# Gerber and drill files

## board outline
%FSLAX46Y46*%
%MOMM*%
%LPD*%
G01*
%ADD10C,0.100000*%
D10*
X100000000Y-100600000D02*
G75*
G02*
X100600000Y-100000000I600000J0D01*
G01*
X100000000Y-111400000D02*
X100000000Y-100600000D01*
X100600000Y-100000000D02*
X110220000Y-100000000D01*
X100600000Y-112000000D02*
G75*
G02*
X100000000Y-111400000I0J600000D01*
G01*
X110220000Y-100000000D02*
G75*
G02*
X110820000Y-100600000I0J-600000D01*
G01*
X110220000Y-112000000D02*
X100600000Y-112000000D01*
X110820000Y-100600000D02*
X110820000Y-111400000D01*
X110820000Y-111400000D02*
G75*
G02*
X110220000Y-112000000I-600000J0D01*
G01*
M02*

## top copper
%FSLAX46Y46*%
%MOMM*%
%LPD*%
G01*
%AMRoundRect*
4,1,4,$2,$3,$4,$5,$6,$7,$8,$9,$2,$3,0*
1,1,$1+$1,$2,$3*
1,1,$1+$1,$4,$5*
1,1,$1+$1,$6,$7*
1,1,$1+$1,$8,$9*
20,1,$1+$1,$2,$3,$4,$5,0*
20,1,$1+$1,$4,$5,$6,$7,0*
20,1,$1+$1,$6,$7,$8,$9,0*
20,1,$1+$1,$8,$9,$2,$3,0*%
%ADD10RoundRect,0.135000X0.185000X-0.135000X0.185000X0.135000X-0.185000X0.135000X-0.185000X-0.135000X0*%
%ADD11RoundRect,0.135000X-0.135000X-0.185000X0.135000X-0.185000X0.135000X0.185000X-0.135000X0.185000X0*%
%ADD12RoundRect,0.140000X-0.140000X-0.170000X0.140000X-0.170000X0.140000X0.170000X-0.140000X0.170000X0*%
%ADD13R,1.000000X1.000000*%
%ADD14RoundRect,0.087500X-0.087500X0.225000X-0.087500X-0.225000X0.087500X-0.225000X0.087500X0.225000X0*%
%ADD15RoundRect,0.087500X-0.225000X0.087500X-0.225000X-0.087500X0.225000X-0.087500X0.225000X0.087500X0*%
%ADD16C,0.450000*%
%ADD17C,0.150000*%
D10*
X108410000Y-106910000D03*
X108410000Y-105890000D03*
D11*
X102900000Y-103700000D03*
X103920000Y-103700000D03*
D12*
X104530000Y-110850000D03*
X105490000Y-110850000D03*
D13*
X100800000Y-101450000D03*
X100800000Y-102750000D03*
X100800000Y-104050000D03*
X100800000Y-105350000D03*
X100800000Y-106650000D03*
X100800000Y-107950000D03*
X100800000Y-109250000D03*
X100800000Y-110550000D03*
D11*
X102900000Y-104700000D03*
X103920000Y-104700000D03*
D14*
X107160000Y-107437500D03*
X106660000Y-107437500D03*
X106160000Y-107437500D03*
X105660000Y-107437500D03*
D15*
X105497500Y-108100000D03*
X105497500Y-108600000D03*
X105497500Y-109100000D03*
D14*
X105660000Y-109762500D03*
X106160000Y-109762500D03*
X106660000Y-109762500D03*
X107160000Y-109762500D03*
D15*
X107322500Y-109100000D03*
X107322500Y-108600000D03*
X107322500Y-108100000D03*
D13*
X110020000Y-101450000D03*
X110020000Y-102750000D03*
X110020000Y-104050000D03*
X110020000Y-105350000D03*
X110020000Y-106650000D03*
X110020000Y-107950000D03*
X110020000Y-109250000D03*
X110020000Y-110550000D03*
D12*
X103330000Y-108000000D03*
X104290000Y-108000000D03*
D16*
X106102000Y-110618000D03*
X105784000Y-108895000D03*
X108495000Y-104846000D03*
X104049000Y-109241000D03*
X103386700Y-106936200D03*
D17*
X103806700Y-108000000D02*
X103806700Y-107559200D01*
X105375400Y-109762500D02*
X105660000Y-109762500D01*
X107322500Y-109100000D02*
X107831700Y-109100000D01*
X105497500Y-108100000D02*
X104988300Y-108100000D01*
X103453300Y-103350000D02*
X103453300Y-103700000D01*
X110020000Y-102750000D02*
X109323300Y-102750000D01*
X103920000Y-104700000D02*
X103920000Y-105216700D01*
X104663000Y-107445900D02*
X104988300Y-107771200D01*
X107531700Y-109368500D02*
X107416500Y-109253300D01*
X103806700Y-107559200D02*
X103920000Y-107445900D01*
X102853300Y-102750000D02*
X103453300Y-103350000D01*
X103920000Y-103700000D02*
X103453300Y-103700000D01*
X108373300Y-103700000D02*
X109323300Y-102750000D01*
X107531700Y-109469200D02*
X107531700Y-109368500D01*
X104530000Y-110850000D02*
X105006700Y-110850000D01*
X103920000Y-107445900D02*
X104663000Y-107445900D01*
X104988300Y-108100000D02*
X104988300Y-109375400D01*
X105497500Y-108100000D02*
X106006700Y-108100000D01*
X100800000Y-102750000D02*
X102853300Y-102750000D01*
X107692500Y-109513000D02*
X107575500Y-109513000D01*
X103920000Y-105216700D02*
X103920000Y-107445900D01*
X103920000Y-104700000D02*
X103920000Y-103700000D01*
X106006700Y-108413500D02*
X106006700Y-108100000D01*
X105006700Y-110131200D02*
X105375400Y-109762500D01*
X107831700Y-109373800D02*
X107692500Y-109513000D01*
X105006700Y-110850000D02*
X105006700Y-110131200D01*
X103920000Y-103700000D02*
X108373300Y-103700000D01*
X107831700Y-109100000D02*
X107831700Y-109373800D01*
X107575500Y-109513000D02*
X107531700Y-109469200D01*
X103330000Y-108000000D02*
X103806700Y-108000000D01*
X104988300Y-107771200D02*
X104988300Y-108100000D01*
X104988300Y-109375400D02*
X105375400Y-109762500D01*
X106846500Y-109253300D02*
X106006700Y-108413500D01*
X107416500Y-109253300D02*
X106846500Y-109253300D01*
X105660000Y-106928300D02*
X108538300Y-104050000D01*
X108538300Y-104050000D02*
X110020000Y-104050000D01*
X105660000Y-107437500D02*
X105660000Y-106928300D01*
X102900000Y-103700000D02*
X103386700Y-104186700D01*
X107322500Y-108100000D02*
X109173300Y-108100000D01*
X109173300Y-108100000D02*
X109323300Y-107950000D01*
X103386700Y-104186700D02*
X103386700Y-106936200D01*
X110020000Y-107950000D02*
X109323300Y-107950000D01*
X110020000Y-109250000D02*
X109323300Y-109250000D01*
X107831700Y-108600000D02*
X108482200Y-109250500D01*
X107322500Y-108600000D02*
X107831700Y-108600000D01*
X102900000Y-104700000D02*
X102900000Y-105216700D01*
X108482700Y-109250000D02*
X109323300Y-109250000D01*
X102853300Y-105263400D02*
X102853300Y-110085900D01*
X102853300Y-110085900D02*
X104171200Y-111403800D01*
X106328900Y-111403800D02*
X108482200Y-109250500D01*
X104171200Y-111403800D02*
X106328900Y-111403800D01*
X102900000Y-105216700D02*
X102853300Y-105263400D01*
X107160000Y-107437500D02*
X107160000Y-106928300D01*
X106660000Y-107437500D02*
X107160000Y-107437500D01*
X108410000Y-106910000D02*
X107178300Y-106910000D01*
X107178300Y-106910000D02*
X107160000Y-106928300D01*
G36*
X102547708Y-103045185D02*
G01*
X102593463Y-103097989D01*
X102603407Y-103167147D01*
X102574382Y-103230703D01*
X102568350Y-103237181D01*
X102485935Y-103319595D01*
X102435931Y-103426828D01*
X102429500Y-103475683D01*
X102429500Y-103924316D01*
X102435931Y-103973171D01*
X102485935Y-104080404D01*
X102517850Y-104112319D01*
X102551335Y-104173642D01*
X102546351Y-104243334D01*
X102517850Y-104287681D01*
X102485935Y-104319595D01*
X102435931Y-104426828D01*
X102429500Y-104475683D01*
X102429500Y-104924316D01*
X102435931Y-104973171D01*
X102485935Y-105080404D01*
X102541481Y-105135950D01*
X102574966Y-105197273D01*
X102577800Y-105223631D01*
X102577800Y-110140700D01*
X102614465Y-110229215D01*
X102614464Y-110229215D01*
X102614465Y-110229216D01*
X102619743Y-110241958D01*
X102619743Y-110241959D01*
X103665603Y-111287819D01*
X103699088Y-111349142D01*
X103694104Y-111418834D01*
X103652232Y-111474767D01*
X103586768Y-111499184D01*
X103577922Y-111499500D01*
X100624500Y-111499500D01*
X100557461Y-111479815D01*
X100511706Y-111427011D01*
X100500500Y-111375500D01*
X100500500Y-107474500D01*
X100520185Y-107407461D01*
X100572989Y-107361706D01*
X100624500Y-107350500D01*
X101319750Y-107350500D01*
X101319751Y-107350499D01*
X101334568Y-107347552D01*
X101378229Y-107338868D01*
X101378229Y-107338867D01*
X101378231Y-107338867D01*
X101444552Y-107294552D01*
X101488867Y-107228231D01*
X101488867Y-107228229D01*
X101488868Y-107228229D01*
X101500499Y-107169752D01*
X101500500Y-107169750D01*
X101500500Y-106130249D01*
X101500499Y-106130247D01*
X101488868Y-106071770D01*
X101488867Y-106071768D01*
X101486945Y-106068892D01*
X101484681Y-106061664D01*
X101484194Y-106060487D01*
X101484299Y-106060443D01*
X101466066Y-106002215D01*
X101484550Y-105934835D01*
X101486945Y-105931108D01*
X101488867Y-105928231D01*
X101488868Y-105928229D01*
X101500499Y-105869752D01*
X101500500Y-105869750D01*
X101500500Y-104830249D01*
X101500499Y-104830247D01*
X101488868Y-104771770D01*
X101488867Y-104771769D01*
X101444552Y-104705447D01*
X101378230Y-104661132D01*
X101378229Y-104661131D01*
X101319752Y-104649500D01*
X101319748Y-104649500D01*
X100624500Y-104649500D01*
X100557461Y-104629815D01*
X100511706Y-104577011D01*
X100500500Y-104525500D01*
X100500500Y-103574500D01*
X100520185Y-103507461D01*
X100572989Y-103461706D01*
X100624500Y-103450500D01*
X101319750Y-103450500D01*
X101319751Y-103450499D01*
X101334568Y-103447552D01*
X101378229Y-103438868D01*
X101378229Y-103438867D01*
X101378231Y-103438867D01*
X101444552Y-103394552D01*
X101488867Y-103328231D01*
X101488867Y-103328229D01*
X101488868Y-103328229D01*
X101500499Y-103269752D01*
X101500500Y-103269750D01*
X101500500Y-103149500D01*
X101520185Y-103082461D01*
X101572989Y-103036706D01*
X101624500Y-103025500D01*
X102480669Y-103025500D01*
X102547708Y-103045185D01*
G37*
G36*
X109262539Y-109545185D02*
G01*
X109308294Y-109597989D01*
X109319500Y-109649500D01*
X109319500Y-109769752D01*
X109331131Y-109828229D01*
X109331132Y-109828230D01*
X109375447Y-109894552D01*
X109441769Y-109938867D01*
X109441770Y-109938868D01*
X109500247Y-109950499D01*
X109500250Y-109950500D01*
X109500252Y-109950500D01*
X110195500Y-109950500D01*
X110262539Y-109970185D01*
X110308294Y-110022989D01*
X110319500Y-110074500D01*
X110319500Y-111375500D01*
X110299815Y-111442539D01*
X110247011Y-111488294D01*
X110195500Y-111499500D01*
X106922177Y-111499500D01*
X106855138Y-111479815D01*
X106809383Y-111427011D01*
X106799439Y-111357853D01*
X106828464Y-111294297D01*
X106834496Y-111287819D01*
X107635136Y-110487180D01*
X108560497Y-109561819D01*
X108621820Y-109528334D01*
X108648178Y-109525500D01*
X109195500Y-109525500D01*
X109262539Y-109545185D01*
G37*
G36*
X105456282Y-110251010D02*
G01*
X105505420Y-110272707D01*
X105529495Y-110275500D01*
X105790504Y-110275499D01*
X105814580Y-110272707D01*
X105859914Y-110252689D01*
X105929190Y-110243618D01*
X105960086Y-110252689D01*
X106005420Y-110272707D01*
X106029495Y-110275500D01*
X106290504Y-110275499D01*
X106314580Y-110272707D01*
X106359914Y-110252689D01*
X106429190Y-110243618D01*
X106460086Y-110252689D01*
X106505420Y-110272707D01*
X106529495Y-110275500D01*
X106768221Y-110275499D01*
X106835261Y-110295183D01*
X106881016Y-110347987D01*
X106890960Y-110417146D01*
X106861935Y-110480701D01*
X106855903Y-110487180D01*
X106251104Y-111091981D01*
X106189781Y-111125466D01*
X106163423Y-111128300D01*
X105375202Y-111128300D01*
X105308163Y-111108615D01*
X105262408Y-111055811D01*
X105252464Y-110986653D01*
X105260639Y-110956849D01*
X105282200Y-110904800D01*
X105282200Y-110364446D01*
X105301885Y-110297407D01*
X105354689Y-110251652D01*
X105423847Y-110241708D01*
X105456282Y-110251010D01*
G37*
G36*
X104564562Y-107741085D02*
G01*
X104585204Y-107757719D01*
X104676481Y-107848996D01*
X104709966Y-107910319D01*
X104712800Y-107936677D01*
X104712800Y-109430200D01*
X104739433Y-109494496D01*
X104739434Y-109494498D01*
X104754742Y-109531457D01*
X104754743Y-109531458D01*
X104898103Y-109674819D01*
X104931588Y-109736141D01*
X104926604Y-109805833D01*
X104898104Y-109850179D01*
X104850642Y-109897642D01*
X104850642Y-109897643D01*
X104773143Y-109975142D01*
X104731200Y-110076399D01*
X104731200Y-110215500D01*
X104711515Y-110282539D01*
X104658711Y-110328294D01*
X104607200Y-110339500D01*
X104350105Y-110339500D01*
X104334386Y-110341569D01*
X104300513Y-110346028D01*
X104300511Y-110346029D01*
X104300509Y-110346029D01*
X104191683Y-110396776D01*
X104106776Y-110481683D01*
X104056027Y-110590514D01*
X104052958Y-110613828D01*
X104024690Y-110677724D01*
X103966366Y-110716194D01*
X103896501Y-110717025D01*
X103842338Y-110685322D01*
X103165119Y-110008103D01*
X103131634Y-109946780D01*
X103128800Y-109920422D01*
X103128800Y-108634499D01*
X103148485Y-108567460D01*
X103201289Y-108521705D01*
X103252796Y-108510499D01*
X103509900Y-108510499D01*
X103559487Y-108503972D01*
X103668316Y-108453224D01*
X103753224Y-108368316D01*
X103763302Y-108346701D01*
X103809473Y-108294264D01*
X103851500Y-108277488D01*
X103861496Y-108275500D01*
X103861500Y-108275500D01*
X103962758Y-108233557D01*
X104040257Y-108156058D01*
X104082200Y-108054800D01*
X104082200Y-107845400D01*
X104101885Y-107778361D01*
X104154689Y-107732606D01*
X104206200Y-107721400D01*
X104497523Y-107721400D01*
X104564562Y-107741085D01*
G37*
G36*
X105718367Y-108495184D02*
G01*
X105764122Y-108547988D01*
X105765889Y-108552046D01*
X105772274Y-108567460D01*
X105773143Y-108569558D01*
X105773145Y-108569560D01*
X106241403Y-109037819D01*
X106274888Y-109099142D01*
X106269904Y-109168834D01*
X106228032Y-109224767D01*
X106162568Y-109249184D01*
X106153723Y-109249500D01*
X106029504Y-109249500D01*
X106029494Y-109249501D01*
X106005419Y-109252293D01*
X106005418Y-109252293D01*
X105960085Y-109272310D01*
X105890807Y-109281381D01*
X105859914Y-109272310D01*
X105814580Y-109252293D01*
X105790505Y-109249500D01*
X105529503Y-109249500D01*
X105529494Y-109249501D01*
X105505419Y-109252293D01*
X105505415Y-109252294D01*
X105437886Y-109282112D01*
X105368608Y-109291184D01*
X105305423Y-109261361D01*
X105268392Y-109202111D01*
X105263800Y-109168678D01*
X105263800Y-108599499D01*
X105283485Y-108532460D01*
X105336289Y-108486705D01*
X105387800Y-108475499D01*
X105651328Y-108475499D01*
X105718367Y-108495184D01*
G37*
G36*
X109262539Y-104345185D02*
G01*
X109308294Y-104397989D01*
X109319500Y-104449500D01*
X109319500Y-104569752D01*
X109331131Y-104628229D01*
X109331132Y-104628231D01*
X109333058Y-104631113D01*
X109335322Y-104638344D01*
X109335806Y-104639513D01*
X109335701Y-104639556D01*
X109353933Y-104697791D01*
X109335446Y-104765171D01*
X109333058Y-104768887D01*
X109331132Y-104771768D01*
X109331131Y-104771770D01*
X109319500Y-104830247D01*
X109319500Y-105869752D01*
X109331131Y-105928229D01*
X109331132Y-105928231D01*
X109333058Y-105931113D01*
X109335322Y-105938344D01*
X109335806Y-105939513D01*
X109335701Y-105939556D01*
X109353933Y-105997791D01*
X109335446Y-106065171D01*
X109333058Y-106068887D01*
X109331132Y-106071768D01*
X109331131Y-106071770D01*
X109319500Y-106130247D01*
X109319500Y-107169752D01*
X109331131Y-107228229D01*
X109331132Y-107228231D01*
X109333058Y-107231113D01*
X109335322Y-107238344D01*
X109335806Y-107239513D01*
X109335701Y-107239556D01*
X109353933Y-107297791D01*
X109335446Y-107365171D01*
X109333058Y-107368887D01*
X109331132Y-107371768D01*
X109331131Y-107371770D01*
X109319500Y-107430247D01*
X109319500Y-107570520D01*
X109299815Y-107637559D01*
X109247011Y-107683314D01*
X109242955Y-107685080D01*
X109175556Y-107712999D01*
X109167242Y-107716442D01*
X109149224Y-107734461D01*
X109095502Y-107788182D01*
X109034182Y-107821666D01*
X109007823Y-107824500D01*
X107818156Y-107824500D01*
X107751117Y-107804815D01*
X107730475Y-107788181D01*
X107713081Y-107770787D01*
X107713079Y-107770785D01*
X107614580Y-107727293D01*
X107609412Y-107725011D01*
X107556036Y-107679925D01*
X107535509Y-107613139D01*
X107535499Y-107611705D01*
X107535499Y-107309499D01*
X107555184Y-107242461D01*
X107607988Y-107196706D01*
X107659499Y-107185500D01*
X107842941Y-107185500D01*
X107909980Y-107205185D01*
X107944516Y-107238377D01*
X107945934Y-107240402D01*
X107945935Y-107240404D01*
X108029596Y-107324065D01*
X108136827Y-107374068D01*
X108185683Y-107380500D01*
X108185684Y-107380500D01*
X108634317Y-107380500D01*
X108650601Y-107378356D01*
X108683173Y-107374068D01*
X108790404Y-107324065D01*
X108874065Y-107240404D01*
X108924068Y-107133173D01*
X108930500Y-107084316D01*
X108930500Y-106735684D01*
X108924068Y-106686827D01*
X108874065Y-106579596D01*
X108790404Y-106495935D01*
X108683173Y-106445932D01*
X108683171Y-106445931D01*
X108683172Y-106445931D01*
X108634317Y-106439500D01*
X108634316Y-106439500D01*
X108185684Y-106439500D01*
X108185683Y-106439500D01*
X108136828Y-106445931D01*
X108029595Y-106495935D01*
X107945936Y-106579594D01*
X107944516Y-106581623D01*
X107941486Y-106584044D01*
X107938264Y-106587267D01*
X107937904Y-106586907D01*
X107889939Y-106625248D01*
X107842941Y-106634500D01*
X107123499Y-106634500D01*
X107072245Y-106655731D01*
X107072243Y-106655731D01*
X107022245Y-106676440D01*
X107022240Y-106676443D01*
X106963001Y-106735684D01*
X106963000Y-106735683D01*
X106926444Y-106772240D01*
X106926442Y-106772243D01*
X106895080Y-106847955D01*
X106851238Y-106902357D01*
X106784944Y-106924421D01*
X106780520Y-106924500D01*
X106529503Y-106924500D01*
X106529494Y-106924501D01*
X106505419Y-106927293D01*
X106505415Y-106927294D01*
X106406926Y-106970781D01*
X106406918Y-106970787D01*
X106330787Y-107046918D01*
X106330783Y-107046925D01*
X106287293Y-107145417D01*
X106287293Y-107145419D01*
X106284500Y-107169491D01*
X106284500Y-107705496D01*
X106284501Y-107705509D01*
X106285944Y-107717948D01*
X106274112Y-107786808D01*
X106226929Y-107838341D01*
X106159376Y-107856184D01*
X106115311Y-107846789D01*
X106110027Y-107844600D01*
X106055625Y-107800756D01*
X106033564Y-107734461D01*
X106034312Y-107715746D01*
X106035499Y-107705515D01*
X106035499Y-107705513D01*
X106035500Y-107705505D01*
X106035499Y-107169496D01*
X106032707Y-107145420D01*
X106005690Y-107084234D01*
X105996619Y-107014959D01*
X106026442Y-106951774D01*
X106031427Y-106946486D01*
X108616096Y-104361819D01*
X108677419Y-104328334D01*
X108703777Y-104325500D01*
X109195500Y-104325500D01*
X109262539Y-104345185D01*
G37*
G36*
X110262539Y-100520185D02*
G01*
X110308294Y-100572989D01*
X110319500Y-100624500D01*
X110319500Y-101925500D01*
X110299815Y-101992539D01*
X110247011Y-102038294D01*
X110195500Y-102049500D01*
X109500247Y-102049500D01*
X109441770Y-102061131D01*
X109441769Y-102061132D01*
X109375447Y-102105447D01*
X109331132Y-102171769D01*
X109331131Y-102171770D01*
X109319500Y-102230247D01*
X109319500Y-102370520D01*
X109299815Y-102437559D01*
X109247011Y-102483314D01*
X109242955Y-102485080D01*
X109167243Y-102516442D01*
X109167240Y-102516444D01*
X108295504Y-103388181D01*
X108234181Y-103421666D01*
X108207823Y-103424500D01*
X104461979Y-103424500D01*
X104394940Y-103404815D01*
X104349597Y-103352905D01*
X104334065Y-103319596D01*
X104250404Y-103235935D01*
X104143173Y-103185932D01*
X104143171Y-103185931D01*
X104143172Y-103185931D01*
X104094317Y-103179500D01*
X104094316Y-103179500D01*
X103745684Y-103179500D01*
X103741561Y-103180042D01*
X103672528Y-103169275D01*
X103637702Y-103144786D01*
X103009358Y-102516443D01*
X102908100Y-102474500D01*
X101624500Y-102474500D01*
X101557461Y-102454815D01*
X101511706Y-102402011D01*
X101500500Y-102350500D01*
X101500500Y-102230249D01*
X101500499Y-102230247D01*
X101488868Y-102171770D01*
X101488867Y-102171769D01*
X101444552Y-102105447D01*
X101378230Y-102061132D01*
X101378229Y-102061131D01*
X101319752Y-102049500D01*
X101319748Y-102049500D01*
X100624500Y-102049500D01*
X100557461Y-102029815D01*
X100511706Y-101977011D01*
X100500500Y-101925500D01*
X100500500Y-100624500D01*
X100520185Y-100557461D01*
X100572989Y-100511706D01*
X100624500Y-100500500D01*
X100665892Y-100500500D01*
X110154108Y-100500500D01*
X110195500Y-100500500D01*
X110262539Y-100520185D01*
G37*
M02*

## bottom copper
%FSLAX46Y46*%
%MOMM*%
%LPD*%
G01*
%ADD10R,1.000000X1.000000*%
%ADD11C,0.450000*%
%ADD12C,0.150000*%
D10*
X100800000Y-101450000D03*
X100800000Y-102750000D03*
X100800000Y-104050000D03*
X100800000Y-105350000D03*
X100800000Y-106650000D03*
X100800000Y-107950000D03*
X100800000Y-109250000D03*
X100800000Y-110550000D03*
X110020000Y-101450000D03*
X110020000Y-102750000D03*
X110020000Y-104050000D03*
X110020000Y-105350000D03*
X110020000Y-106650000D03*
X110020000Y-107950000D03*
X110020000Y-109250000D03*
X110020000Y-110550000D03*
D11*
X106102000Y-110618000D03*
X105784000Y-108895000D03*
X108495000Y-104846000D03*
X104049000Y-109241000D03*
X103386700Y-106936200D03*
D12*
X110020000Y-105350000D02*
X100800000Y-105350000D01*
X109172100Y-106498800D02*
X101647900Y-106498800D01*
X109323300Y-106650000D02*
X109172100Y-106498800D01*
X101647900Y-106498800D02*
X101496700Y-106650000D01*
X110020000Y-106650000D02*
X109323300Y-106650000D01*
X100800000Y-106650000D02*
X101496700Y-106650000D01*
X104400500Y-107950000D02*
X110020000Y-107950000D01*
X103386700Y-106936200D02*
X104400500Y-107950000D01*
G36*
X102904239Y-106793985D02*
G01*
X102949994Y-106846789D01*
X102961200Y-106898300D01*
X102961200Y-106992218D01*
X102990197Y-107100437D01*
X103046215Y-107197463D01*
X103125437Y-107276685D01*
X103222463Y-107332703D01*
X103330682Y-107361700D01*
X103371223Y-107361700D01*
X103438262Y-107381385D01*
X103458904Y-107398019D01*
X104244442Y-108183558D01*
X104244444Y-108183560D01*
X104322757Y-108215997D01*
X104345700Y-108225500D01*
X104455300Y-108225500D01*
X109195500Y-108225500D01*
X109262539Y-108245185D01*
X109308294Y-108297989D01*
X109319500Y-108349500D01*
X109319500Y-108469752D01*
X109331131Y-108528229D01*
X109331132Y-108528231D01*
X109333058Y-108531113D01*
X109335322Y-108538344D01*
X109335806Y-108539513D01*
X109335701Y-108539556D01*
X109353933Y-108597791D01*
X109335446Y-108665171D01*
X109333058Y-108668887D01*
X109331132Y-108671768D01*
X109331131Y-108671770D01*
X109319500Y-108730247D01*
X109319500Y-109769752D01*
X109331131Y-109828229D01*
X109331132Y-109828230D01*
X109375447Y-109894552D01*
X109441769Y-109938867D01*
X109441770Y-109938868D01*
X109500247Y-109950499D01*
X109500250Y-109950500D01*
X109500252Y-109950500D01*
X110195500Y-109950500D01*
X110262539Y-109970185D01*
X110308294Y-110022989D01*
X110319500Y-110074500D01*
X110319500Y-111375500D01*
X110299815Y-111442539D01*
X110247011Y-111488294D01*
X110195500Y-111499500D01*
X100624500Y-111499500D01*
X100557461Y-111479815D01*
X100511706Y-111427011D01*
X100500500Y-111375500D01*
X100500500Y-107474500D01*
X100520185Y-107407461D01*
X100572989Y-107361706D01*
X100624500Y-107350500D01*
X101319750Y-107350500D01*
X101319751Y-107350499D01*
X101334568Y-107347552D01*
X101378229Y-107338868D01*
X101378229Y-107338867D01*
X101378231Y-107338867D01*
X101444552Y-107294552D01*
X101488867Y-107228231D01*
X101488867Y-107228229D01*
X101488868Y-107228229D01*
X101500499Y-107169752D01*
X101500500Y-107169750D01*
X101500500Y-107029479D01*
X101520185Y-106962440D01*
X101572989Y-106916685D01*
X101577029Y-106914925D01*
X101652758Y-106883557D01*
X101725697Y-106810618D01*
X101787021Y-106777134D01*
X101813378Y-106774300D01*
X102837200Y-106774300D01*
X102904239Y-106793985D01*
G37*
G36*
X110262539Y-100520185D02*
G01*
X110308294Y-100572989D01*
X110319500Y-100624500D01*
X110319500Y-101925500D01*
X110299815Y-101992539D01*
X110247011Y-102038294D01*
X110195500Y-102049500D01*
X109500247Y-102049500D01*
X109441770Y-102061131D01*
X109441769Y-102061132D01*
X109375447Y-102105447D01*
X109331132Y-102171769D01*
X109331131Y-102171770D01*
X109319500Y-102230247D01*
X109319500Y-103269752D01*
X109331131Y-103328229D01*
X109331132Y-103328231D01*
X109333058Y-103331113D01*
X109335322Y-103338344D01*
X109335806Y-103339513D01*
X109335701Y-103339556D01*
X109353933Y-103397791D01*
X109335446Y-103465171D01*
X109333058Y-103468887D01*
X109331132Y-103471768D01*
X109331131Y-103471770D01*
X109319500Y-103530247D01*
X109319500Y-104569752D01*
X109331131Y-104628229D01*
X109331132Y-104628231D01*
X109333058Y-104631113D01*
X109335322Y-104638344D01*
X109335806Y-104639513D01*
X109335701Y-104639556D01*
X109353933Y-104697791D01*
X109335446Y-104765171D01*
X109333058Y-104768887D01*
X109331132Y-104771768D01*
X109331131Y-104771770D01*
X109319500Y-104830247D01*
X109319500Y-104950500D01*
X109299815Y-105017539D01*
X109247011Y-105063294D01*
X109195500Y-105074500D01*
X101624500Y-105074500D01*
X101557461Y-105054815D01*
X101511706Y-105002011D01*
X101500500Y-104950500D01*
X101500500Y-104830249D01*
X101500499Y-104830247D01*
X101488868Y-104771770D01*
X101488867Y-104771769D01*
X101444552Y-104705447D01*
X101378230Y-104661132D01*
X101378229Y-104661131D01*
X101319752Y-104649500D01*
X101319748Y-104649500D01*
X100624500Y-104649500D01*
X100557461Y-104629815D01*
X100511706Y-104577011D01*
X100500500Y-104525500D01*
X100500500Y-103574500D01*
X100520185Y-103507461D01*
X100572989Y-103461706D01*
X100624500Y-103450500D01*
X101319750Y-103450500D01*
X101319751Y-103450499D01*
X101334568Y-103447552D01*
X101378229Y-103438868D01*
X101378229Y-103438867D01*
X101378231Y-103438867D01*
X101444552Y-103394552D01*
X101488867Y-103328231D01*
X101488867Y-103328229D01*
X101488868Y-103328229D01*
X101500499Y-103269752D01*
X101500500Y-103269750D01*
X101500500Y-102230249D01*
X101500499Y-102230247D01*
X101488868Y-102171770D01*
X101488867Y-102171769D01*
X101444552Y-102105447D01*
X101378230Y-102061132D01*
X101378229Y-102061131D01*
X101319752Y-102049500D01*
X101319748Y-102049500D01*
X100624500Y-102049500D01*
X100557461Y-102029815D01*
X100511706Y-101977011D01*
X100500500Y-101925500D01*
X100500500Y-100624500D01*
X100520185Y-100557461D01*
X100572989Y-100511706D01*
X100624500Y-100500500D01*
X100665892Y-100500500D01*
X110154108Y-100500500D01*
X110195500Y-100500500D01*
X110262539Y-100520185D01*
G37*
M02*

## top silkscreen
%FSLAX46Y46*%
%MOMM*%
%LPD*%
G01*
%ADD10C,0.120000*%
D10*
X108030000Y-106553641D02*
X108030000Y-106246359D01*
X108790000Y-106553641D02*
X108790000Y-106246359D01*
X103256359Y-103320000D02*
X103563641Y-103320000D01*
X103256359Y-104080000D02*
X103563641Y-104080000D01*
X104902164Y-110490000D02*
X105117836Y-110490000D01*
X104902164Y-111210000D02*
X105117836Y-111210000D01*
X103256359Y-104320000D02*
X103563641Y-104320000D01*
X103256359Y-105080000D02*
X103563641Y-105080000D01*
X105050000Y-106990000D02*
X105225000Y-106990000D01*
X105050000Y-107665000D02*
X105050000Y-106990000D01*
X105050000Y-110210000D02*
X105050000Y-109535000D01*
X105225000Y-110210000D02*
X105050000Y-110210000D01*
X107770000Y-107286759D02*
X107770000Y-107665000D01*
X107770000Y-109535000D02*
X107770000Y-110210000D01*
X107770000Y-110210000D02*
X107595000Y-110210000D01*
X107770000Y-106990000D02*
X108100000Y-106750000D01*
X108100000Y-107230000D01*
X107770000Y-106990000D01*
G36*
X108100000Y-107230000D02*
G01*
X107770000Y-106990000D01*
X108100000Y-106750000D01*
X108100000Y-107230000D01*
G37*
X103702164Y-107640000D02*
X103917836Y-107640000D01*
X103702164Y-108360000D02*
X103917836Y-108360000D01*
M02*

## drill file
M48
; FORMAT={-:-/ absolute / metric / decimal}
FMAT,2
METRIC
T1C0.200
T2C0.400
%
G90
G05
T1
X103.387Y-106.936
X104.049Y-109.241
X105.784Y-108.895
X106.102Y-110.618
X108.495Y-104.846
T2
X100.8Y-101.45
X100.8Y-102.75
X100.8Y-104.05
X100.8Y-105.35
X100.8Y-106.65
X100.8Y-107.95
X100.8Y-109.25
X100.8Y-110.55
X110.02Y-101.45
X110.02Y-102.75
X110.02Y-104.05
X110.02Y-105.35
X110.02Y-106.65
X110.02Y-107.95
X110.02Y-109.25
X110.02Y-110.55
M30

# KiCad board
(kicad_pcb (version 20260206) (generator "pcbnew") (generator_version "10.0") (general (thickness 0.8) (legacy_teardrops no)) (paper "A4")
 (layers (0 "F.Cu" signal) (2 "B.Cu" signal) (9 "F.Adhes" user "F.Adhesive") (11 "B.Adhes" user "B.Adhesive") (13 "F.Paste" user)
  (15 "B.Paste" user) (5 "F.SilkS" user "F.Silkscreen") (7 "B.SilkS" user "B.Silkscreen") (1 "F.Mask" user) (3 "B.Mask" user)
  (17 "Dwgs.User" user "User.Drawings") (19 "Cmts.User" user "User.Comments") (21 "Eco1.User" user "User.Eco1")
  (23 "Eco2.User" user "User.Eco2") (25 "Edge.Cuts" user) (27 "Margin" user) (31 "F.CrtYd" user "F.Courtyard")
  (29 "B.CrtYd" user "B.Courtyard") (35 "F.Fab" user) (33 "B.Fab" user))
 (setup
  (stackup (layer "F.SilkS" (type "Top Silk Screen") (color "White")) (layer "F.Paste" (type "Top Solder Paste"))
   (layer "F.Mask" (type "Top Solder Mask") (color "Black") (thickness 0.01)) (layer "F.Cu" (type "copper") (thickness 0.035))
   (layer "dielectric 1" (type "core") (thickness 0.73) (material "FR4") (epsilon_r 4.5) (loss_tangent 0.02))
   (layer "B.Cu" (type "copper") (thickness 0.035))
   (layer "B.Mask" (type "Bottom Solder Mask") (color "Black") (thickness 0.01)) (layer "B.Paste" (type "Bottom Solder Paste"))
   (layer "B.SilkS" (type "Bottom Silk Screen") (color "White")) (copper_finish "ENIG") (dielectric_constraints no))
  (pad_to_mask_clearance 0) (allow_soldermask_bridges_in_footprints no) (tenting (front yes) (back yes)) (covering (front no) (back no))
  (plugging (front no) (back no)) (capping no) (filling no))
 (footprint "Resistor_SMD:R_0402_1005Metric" (layer "F.Cu") (at 108.41 106.4 90)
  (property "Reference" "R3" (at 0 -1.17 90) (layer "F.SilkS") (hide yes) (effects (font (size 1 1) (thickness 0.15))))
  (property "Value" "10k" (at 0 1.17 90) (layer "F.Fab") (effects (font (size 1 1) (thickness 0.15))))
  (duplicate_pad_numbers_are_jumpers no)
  (fp_line (start -0.153641 -0.38) (end 0.153641 -0.38) (stroke (width 0.12) (type solid)) (layer "F.SilkS"))
  (fp_line (start -0.153641 0.38) (end 0.153641 0.38) (stroke (width 0.12) (type solid)) (layer "F.SilkS"))
  (pad "1" smd roundrect (at -0.51 0 90) (size 0.54 0.64) (layers "F.Cu" "F.Mask" "F.Paste") (roundrect_rratio 0.25) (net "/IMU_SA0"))
  (pad "2" smd roundrect (at 0.51 0 90) (size 0.54 0.64) (layers "F.Cu" "F.Mask" "F.Paste") (roundrect_rratio 0.25) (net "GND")))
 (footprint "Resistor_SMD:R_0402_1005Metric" (layer "F.Cu") (at 103.41 103.7)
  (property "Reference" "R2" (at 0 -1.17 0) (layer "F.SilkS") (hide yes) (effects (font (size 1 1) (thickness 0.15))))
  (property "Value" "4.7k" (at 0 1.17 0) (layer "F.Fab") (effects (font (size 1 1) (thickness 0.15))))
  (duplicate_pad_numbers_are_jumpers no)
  (fp_line (start -0.153641 -0.38) (end 0.153641 -0.38) (stroke (width 0.12) (type solid)) (layer "F.SilkS"))
  (fp_line (start -0.153641 0.38) (end 0.153641 0.38) (stroke (width 0.12) (type solid)) (layer "F.SilkS"))
  (pad "1" smd roundrect (at -0.51 0) (size 0.54 0.64) (layers "F.Cu" "F.Mask" "F.Paste") (roundrect_rratio 0.25) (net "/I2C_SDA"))
  (pad "2" smd roundrect (at 0.51 0) (size 0.54 0.64) (layers "F.Cu" "F.Mask" "F.Paste") (roundrect_rratio 0.25) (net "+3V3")))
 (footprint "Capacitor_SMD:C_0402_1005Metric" (layer "F.Cu") (at 105.01 110.85)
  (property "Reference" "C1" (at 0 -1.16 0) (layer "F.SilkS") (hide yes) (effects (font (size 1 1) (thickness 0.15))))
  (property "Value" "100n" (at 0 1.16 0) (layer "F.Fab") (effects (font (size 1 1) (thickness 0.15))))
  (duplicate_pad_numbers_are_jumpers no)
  (fp_line (start -0.107836 -0.36) (end 0.107836 -0.36) (stroke (width 0.12) (type solid)) (layer "F.SilkS"))
  (fp_line (start -0.107836 0.36) (end 0.107836 0.36) (stroke (width 0.12) (type solid)) (layer "F.SilkS"))
  (pad "1" smd roundrect (at -0.48 0) (size 0.56 0.62) (layers "F.Cu" "F.Mask" "F.Paste") (roundrect_rratio 0.25) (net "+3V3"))
  (pad "2" smd roundrect (at 0.48 0) (size 0.56 0.62) (layers "F.Cu" "F.Mask" "F.Paste") (roundrect_rratio 0.25) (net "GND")))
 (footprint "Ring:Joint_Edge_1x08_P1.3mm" (layer "F.Cu") (at 100.8 106)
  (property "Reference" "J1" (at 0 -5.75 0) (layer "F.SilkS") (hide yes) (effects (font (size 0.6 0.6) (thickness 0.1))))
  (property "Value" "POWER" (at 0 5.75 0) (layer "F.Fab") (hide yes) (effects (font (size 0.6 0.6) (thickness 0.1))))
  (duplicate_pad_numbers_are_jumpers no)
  (pad "1" thru_hole rect (at 0 -4.55) (size 1 1) (drill 0.4) (layers "*.Cu" "*.Mask") (remove_unused_layers no) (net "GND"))
  (pad "2" thru_hole rect (at 0 -3.25) (size 1 1) (drill 0.4) (layers "*.Cu" "*.Mask") (remove_unused_layers no) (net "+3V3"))
  (pad "3" thru_hole rect (at 0 -1.95) (size 1 1) (drill 0.4) (layers "*.Cu" "*.Mask") (remove_unused_layers no) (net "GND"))
  (pad "4" thru_hole rect (at 0 -0.65) (size 1 1) (drill 0.4) (layers "*.Cu" "*.Mask") (remove_unused_layers no) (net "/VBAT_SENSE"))
  (pad "5" thru_hole rect (at 0 0.65) (size 1 1) (drill 0.4) (layers "*.Cu" "*.Mask") (remove_unused_layers no) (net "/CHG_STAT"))
  (pad "6" thru_hole rect (at 0 1.95) (size 1 1) (drill 0.4) (layers "*.Cu" "*.Mask") (remove_unused_layers no) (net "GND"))
  (pad "7" thru_hole rect (at 0 3.25) (size 1 1) (drill 0.4) (layers "*.Cu" "*.Mask") (remove_unused_layers no) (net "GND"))
  (pad "8" thru_hole rect (at 0 4.55) (size 1 1) (drill 0.4) (layers "*.Cu" "*.Mask") (remove_unused_layers no) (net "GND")))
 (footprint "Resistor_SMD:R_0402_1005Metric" (layer "F.Cu") (at 103.41 104.7)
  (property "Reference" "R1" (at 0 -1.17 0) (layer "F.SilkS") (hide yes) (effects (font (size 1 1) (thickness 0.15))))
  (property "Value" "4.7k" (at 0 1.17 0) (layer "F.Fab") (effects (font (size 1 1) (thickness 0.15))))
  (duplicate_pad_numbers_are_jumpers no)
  (fp_line (start -0.153641 -0.38) (end 0.153641 -0.38) (stroke (width 0.12) (type solid)) (layer "F.SilkS"))
  (fp_line (start -0.153641 0.38) (end 0.153641 0.38) (stroke (width 0.12) (type solid)) (layer "F.SilkS"))
  (pad "1" smd roundrect (at -0.51 0) (size 0.54 0.64) (layers "F.Cu" "F.Mask" "F.Paste") (roundrect_rratio 0.25) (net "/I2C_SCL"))
  (pad "2" smd roundrect (at 0.51 0) (size 0.54 0.64) (layers "F.Cu" "F.Mask" "F.Paste") (roundrect_rratio 0.25) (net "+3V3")))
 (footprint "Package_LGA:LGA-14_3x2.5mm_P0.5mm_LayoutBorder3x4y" (layer "F.Cu") (at 106.41 108.6 -90)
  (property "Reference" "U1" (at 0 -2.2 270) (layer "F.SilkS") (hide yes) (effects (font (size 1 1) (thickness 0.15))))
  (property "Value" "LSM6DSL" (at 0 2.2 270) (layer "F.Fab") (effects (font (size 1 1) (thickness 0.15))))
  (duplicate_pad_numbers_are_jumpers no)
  (fp_line (start -1.61 1.36) (end -1.61 1.185) (stroke (width 0.12) (type solid)) (layer "F.SilkS"))
  (fp_line (start -0.935 1.36) (end -1.61 1.36) (stroke (width 0.12) (type solid)) (layer "F.SilkS"))
  (fp_line (start 1.61 1.36) (end 0.935 1.36) (stroke (width 0.12) (type solid)) (layer "F.SilkS"))
  (fp_line (start 1.61 1.185) (end 1.61 1.36) (stroke (width 0.12) (type solid)) (layer "F.SilkS"))
  (fp_line (start -1.313241 -1.36) (end -0.935 -1.36) (stroke (width 0.12) (type solid)) (layer "F.SilkS"))
  (fp_line (start 0.935 -1.36) (end 1.61 -1.36) (stroke (width 0.12) (type solid)) (layer "F.SilkS"))
  (fp_line (start 1.61 -1.36) (end 1.61 -1.185) (stroke (width 0.12) (type solid)) (layer "F.SilkS"))
  (fp_poly (pts (xy -1.61 -1.36) (xy -1.85 -1.69) (xy -1.37 -1.69)) (stroke (width 0.12) (type solid)) (fill yes) (layer "F.SilkS"))
  (pad "1" smd roundrect (at -1.1625 -0.75 270) (size 0.625 0.35) (layers "F.Cu" "F.Mask" "F.Paste") (roundrect_rratio 0.25)
   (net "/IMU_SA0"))
  (pad "2" smd roundrect (at -1.1625 -0.25 270) (size 0.625 0.35) (layers "F.Cu" "F.Mask" "F.Paste") (roundrect_rratio 0.25)
   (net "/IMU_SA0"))
  (pad "3" smd roundrect (at -1.1625 0.25 270) (size 0.625 0.35) (layers "F.Cu" "F.Mask" "F.Paste") (roundrect_rratio 0.25) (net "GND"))
  (pad "4" smd roundrect (at -1.1625 0.75 270) (size 0.625 0.35) (layers "F.Cu" "F.Mask" "F.Paste") (roundrect_rratio 0.25) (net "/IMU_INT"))
  (pad "5" smd roundrect (at -0.5 0.9125 270) (size 0.35 0.625) (layers "F.Cu" "F.Mask" "F.Paste") (roundrect_rratio 0.25) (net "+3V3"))
  (pad "6" smd roundrect (at 0 0.9125 270) (size 0.35 0.625) (layers "F.Cu" "F.Mask" "F.Paste") (roundrect_rratio 0.25) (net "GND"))
  (pad "7" smd roundrect (at 0.5 0.9125 270) (size 0.35 0.625) (layers "F.Cu" "F.Mask" "F.Paste") (roundrect_rratio 0.25) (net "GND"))
  (pad "8" smd roundrect (at 1.1625 0.75 270) (size 0.625 0.35) (layers "F.Cu" "F.Mask" "F.Paste") (roundrect_rratio 0.25) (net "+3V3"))
  (pad "9" smd roundrect (at 1.1625 0.25 270) (size 0.625 0.35) (layers "F.Cu" "F.Mask" "F.Paste") (roundrect_rratio 0.25)
   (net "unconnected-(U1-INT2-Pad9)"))
  (pad "10" smd roundrect (at 1.1625 -0.25 270) (size 0.625 0.35) (layers "F.Cu" "F.Mask" "F.Paste") (roundrect_rratio 0.25)
   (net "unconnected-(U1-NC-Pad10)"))
  (pad "11" smd roundrect (at 1.1625 -0.75 270) (size 0.625 0.35) (layers "F.Cu" "F.Mask" "F.Paste") (roundrect_rratio 0.25)
   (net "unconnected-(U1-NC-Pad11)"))
  (pad "12" smd roundrect (at 0.5 -0.9125 270) (size 0.35 0.625) (layers "F.Cu" "F.Mask" "F.Paste") (roundrect_rratio 0.25) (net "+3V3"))
  (pad "13" smd roundrect (at 0 -0.9125 270) (size 0.35 0.625) (layers "F.Cu" "F.Mask" "F.Paste") (roundrect_rratio 0.25) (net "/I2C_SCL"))
  (pad "14" smd roundrect (at -0.5 -0.9125 270) (size 0.35 0.625) (layers "F.Cu" "F.Mask" "F.Paste") (roundrect_rratio 0.25)
   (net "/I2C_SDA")))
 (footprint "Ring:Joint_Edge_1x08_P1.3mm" (layer "F.Cu") (at 110.02 106)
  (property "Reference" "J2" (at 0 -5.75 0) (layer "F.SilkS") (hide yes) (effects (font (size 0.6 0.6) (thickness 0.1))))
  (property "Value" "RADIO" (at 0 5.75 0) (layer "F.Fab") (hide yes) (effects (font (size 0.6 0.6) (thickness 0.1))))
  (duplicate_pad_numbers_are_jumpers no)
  (pad "1" thru_hole rect (at 0 -4.55) (size 1 1) (drill 0.4) (layers "*.Cu" "*.Mask") (remove_unused_layers no) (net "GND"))
  (pad "2" thru_hole rect (at 0 -3.25) (size 1 1) (drill 0.4) (layers "*.Cu" "*.Mask") (remove_unused_layers no) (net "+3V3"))
  (pad "3" thru_hole rect (at 0 -1.95) (size 1 1) (drill 0.4) (layers "*.Cu" "*.Mask") (remove_unused_layers no) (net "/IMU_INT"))
  (pad "4" thru_hole rect (at 0 -0.65) (size 1 1) (drill 0.4) (layers "*.Cu" "*.Mask") (remove_unused_layers no) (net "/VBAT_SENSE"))
  (pad "5" thru_hole rect (at 0 0.65) (size 1 1) (drill 0.4) (layers "*.Cu" "*.Mask") (remove_unused_layers no) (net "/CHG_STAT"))
  (pad "6" thru_hole rect (at 0 1.95) (size 1 1) (drill 0.4) (layers "*.Cu" "*.Mask") (remove_unused_layers no) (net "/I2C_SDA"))
  (pad "7" thru_hole rect (at 0 3.25) (size 1 1) (drill 0.4) (layers "*.Cu" "*.Mask") (remove_unused_layers no) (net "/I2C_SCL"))
  (pad "8" thru_hole rect (at 0 4.55) (size 1 1) (drill 0.4) (layers "*.Cu" "*.Mask") (remove_unused_layers no) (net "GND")))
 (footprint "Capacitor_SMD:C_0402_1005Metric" (layer "F.Cu") (at 103.81 108)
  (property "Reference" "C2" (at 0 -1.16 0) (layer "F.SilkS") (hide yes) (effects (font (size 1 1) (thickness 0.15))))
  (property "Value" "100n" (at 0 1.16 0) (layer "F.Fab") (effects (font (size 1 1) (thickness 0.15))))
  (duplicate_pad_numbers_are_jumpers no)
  (fp_line (start -0.107836 -0.36) (end 0.107836 -0.36) (stroke (width 0.12) (type solid)) (layer "F.SilkS"))
  (fp_line (start -0.107836 0.36) (end 0.107836 0.36) (stroke (width 0.12) (type solid)) (layer "F.SilkS"))
  (pad "1" smd roundrect (at -0.48 0) (size 0.56 0.62) (layers "F.Cu" "F.Mask" "F.Paste") (roundrect_rratio 0.25) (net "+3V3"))
  (pad "2" smd roundrect (at 0.48 0) (size 0.56 0.62) (layers "F.Cu" "F.Mask" "F.Paste") (roundrect_rratio 0.25) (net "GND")))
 (gr_arc (start 100 100.6) (mid 100.175736 100.175736) (end 100.6 100) (stroke (width 0.1) (type default)) (layer "Edge.Cuts"))
 (gr_line (start 100 111.4) (end 100 100.6) (stroke (width 0.1) (type default)) (layer "Edge.Cuts"))
 (gr_line (start 100.6 100) (end 110.22 100) (stroke (width 0.1) (type default)) (layer "Edge.Cuts"))
 (gr_arc (start 100.6 112) (mid 100.175736 111.824264) (end 100 111.4) (stroke (width 0.1) (type default)) (layer "Edge.Cuts"))
 (gr_arc (start 110.22 100) (mid 110.644264 100.175736) (end 110.82 100.6) (stroke (width 0.1) (type default)) (layer "Edge.Cuts"))
 (gr_line (start 110.22 112) (end 100.6 112) (stroke (width 0.1) (type default)) (layer "Edge.Cuts"))
 (gr_line (start 110.82 100.6) (end 110.82 111.4) (stroke (width 0.1) (type default)) (layer "Edge.Cuts"))
 (gr_arc (start 110.82 111.4) (mid 110.644264 111.824264) (end 110.22 112) (stroke (width 0.1) (type default)) (layer "Edge.Cuts"))
 (via (at 106.102 110.618) (size 0.45) (drill 0.2) (layers "F.Cu" "B.Cu") (capping no) (covering (front no) (back no))
  (plugging (front no) (back no)) (filling no) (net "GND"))
 (via (at 105.784 108.895) (size 0.45) (drill 0.2) (layers "F.Cu" "B.Cu") (capping no) (covering (front no) (back no))
  (plugging (front no) (back no)) (filling no) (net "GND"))
 (via (at 108.495 104.846) (size 0.45) (drill 0.2) (layers "F.Cu" "B.Cu") (capping no) (covering (front no) (back no))
  (plugging (front no) (back no)) (filling no) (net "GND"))
 (via (at 104.049 109.241) (size 0.45) (drill 0.2) (layers "F.Cu" "B.Cu") (capping no) (covering (front no) (back no))
  (plugging (front no) (back no)) (filling no) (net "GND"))
 (segment (start 103.8067 108) (end 103.8067 107.5592) (width 0.15) (layer "F.Cu") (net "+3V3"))
 (segment (start 105.3754 109.7625) (end 105.66 109.7625) (width 0.15) (layer "F.Cu") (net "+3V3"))
 (segment (start 107.3225 109.1) (end 107.8317 109.1) (width 0.15) (layer "F.Cu") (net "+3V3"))
 (segment (start 105.4975 108.1) (end 104.9883 108.1) (width 0.15) (layer "F.Cu") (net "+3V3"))
 (segment (start 103.4533 103.35) (end 103.4533 103.7) (width 0.15) (layer "F.Cu") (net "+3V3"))
 (segment (start 110.02 102.75) (end 109.3233 102.75) (width 0.15) (layer "F.Cu") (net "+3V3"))
 (segment (start 103.92 104.7) (end 103.92 105.2167) (width 0.15) (layer "F.Cu") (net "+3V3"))
 (segment (start 104.663 107.4459) (end 104.9883 107.7712) (width 0.15) (layer "F.Cu") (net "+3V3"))
 (segment (start 107.5317 109.3685) (end 107.4165 109.2533) (width 0.15) (layer "F.Cu") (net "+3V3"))
 (segment (start 103.8067 107.5592) (end 103.92 107.4459) (width 0.15) (layer "F.Cu") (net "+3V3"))
 (segment (start 102.8533 102.75) (end 103.4533 103.35) (width 0.15) (layer "F.Cu") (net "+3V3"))
 (segment (start 103.92 103.7) (end 103.4533 103.7) (width 0.15) (layer "F.Cu") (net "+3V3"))
 (segment (start 108.3733 103.7) (end 109.3233 102.75) (width 0.15) (layer "F.Cu") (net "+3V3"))
 (segment (start 107.5317 109.4692) (end 107.5317 109.3685) (width 0.15) (layer "F.Cu") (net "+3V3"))
 (segment (start 104.53 110.85) (end 105.0067 110.85) (width 0.15) (layer "F.Cu") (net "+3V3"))
 (segment (start 103.92 107.4459) (end 104.663 107.4459) (width 0.15) (layer "F.Cu") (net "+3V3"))
 (segment (start 104.9883 108.1) (end 104.9883 109.3754) (width 0.15) (layer "F.Cu") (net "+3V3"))
 (segment (start 105.4975 108.1) (end 106.0067 108.1) (width 0.15) (layer "F.Cu") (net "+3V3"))
 (segment (start 100.8 102.75) (end 102.8533 102.75) (width 0.15) (layer "F.Cu") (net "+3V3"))
 (segment (start 107.6925 109.513) (end 107.5755 109.513) (width 0.15) (layer "F.Cu") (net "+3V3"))
 (segment (start 103.92 105.2167) (end 103.92 107.4459) (width 0.15) (layer "F.Cu") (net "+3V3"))
 (segment (start 103.92 104.7) (end 103.92 103.7) (width 0.15) (layer "F.Cu") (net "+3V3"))
 (segment (start 106.0067 108.4135) (end 106.0067 108.1) (width 0.15) (layer "F.Cu") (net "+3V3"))
 (segment (start 105.0067 110.1312) (end 105.3754 109.7625) (width 0.15) (layer "F.Cu") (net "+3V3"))
 (segment (start 107.8317 109.3738) (end 107.6925 109.513) (width 0.15) (layer "F.Cu") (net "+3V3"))
 (segment (start 105.0067 110.85) (end 105.0067 110.1312) (width 0.15) (layer "F.Cu") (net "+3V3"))
 (segment (start 103.92 103.7) (end 108.3733 103.7) (width 0.15) (layer "F.Cu") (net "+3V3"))
 (segment (start 107.8317 109.1) (end 107.8317 109.3738) (width 0.15) (layer "F.Cu") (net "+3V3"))
 (segment (start 107.5755 109.513) (end 107.5317 109.4692) (width 0.15) (layer "F.Cu") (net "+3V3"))
 (segment (start 103.33 108) (end 103.8067 108) (width 0.15) (layer "F.Cu") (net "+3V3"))
 (segment (start 104.9883 107.7712) (end 104.9883 108.1) (width 0.15) (layer "F.Cu") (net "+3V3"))
 (segment (start 104.9883 109.3754) (end 105.3754 109.7625) (width 0.15) (layer "F.Cu") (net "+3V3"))
 (segment (start 106.8465 109.2533) (end 106.0067 108.4135) (width 0.15) (layer "F.Cu") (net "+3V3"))
 (segment (start 107.4165 109.2533) (end 106.8465 109.2533) (width 0.15) (layer "F.Cu") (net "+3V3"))
 (segment (start 110.02 105.35) (end 100.8 105.35) (width 0.15) (layer "B.Cu") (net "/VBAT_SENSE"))
 (segment (start 109.1721 106.4988) (end 101.6479 106.4988) (width 0.15) (layer "B.Cu") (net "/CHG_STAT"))
 (segment (start 109.3233 106.65) (end 109.1721 106.4988) (width 0.15) (layer "B.Cu") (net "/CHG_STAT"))
 (segment (start 101.6479 106.4988) (end 101.4967 106.65) (width 0.15) (layer "B.Cu") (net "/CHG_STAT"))
 (segment (start 110.02 106.65) (end 109.3233 106.65) (width 0.15) (layer "B.Cu") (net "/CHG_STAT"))
 (segment (start 100.8 106.65) (end 101.4967 106.65) (width 0.15) (layer "B.Cu") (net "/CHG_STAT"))
 (segment (start 105.66 106.9283) (end 108.5383 104.05) (width 0.15) (layer "F.Cu") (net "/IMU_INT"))
 (segment (start 108.5383 104.05) (end 110.02 104.05) (width 0.15) (layer "F.Cu") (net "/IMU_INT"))
 (segment (start 105.66 107.4375) (end 105.66 106.9283) (width 0.15) (layer "F.Cu") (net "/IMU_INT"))
 (segment (start 102.9 103.7) (end 103.3867 104.1867) (width 0.15) (layer "F.Cu") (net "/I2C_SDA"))
 (segment (start 107.3225 108.1) (end 109.1733 108.1) (width 0.15) (layer "F.Cu") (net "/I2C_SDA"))
 (segment (start 109.1733 108.1) (end 109.3233 107.95) (width 0.15) (layer "F.Cu") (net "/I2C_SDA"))
 (segment (start 103.3867 104.1867) (end 103.3867 106.9362) (width 0.15) (layer "F.Cu") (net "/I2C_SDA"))
 (segment (start 110.02 107.95) (end 109.3233 107.95) (width 0.15) (layer "F.Cu") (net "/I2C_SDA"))
 (via (at 103.3867 106.9362) (size 0.45) (drill 0.2) (layers "F.Cu" "B.Cu") (capping no) (covering (front no) (back no))
  (plugging (front no) (back no)) (filling no) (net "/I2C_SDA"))
 (segment (start 104.4005 107.95) (end 110.02 107.95) (width 0.15) (layer "B.Cu") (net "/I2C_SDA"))
 (segment (start 103.3867 106.9362) (end 104.4005 107.95) (width 0.15) (layer "B.Cu") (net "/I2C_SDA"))
 (segment (start 110.02 109.25) (end 109.3233 109.25) (width 0.15) (layer "F.Cu") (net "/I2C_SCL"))
 (segment (start 107.8317 108.6) (end 108.4822 109.2505) (width 0.15) (layer "F.Cu") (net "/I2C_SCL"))
 (segment (start 107.3225 108.6) (end 107.8317 108.6) (width 0.15) (layer "F.Cu") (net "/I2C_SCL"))
 (segment (start 102.9 104.7) (end 102.9 105.2167) (width 0.15) (layer "F.Cu") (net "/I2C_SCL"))
 (segment (start 108.4827 109.25) (end 109.3233 109.25) (width 0.15) (layer "F.Cu") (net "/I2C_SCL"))
 (segment (start 102.8533 105.2634) (end 102.8533 110.0859) (width 0.15) (layer "F.Cu") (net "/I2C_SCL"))
 (segment (start 102.8533 110.0859) (end 104.1712 111.4038) (width 0.15) (layer "F.Cu") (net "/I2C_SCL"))
 (segment (start 106.3289 111.4038) (end 108.4822 109.2505) (width 0.15) (layer "F.Cu") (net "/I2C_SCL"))
 (segment (start 104.1712 111.4038) (end 106.3289 111.4038) (width 0.15) (layer "F.Cu") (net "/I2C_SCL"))
 (segment (start 102.9 105.2167) (end 102.8533 105.2634) (width 0.15) (layer "F.Cu") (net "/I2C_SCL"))
 (segment (start 107.16 107.4375) (end 107.16 106.9283) (width 0.15) (layer "F.Cu") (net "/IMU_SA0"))
 (segment (start 106.66 107.4375) (end 107.16 107.4375) (width 0.15) (layer "F.Cu") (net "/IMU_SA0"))
 (segment (start 108.41 106.91) (end 107.1783 106.91) (width 0.15) (layer "F.Cu") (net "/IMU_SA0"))
 (segment (start 107.1783 106.91) (end 107.16 106.9283) (width 0.15) (layer "F.Cu") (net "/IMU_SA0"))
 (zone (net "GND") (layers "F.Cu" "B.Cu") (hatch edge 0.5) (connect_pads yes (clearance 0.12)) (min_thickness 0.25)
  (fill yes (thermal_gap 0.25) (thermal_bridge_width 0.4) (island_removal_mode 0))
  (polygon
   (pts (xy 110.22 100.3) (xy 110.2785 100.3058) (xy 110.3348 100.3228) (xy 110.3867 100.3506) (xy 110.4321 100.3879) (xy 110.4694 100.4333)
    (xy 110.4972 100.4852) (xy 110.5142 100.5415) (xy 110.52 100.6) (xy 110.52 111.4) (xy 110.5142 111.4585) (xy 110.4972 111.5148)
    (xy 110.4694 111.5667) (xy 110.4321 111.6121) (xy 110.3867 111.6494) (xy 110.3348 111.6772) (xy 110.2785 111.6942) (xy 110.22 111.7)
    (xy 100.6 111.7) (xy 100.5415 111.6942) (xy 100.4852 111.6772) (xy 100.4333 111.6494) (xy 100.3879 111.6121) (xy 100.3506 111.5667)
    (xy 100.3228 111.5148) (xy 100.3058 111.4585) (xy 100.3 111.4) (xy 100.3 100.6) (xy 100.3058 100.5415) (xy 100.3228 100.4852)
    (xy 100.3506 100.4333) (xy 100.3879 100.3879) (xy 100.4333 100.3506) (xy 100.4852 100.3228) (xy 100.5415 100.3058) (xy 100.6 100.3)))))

